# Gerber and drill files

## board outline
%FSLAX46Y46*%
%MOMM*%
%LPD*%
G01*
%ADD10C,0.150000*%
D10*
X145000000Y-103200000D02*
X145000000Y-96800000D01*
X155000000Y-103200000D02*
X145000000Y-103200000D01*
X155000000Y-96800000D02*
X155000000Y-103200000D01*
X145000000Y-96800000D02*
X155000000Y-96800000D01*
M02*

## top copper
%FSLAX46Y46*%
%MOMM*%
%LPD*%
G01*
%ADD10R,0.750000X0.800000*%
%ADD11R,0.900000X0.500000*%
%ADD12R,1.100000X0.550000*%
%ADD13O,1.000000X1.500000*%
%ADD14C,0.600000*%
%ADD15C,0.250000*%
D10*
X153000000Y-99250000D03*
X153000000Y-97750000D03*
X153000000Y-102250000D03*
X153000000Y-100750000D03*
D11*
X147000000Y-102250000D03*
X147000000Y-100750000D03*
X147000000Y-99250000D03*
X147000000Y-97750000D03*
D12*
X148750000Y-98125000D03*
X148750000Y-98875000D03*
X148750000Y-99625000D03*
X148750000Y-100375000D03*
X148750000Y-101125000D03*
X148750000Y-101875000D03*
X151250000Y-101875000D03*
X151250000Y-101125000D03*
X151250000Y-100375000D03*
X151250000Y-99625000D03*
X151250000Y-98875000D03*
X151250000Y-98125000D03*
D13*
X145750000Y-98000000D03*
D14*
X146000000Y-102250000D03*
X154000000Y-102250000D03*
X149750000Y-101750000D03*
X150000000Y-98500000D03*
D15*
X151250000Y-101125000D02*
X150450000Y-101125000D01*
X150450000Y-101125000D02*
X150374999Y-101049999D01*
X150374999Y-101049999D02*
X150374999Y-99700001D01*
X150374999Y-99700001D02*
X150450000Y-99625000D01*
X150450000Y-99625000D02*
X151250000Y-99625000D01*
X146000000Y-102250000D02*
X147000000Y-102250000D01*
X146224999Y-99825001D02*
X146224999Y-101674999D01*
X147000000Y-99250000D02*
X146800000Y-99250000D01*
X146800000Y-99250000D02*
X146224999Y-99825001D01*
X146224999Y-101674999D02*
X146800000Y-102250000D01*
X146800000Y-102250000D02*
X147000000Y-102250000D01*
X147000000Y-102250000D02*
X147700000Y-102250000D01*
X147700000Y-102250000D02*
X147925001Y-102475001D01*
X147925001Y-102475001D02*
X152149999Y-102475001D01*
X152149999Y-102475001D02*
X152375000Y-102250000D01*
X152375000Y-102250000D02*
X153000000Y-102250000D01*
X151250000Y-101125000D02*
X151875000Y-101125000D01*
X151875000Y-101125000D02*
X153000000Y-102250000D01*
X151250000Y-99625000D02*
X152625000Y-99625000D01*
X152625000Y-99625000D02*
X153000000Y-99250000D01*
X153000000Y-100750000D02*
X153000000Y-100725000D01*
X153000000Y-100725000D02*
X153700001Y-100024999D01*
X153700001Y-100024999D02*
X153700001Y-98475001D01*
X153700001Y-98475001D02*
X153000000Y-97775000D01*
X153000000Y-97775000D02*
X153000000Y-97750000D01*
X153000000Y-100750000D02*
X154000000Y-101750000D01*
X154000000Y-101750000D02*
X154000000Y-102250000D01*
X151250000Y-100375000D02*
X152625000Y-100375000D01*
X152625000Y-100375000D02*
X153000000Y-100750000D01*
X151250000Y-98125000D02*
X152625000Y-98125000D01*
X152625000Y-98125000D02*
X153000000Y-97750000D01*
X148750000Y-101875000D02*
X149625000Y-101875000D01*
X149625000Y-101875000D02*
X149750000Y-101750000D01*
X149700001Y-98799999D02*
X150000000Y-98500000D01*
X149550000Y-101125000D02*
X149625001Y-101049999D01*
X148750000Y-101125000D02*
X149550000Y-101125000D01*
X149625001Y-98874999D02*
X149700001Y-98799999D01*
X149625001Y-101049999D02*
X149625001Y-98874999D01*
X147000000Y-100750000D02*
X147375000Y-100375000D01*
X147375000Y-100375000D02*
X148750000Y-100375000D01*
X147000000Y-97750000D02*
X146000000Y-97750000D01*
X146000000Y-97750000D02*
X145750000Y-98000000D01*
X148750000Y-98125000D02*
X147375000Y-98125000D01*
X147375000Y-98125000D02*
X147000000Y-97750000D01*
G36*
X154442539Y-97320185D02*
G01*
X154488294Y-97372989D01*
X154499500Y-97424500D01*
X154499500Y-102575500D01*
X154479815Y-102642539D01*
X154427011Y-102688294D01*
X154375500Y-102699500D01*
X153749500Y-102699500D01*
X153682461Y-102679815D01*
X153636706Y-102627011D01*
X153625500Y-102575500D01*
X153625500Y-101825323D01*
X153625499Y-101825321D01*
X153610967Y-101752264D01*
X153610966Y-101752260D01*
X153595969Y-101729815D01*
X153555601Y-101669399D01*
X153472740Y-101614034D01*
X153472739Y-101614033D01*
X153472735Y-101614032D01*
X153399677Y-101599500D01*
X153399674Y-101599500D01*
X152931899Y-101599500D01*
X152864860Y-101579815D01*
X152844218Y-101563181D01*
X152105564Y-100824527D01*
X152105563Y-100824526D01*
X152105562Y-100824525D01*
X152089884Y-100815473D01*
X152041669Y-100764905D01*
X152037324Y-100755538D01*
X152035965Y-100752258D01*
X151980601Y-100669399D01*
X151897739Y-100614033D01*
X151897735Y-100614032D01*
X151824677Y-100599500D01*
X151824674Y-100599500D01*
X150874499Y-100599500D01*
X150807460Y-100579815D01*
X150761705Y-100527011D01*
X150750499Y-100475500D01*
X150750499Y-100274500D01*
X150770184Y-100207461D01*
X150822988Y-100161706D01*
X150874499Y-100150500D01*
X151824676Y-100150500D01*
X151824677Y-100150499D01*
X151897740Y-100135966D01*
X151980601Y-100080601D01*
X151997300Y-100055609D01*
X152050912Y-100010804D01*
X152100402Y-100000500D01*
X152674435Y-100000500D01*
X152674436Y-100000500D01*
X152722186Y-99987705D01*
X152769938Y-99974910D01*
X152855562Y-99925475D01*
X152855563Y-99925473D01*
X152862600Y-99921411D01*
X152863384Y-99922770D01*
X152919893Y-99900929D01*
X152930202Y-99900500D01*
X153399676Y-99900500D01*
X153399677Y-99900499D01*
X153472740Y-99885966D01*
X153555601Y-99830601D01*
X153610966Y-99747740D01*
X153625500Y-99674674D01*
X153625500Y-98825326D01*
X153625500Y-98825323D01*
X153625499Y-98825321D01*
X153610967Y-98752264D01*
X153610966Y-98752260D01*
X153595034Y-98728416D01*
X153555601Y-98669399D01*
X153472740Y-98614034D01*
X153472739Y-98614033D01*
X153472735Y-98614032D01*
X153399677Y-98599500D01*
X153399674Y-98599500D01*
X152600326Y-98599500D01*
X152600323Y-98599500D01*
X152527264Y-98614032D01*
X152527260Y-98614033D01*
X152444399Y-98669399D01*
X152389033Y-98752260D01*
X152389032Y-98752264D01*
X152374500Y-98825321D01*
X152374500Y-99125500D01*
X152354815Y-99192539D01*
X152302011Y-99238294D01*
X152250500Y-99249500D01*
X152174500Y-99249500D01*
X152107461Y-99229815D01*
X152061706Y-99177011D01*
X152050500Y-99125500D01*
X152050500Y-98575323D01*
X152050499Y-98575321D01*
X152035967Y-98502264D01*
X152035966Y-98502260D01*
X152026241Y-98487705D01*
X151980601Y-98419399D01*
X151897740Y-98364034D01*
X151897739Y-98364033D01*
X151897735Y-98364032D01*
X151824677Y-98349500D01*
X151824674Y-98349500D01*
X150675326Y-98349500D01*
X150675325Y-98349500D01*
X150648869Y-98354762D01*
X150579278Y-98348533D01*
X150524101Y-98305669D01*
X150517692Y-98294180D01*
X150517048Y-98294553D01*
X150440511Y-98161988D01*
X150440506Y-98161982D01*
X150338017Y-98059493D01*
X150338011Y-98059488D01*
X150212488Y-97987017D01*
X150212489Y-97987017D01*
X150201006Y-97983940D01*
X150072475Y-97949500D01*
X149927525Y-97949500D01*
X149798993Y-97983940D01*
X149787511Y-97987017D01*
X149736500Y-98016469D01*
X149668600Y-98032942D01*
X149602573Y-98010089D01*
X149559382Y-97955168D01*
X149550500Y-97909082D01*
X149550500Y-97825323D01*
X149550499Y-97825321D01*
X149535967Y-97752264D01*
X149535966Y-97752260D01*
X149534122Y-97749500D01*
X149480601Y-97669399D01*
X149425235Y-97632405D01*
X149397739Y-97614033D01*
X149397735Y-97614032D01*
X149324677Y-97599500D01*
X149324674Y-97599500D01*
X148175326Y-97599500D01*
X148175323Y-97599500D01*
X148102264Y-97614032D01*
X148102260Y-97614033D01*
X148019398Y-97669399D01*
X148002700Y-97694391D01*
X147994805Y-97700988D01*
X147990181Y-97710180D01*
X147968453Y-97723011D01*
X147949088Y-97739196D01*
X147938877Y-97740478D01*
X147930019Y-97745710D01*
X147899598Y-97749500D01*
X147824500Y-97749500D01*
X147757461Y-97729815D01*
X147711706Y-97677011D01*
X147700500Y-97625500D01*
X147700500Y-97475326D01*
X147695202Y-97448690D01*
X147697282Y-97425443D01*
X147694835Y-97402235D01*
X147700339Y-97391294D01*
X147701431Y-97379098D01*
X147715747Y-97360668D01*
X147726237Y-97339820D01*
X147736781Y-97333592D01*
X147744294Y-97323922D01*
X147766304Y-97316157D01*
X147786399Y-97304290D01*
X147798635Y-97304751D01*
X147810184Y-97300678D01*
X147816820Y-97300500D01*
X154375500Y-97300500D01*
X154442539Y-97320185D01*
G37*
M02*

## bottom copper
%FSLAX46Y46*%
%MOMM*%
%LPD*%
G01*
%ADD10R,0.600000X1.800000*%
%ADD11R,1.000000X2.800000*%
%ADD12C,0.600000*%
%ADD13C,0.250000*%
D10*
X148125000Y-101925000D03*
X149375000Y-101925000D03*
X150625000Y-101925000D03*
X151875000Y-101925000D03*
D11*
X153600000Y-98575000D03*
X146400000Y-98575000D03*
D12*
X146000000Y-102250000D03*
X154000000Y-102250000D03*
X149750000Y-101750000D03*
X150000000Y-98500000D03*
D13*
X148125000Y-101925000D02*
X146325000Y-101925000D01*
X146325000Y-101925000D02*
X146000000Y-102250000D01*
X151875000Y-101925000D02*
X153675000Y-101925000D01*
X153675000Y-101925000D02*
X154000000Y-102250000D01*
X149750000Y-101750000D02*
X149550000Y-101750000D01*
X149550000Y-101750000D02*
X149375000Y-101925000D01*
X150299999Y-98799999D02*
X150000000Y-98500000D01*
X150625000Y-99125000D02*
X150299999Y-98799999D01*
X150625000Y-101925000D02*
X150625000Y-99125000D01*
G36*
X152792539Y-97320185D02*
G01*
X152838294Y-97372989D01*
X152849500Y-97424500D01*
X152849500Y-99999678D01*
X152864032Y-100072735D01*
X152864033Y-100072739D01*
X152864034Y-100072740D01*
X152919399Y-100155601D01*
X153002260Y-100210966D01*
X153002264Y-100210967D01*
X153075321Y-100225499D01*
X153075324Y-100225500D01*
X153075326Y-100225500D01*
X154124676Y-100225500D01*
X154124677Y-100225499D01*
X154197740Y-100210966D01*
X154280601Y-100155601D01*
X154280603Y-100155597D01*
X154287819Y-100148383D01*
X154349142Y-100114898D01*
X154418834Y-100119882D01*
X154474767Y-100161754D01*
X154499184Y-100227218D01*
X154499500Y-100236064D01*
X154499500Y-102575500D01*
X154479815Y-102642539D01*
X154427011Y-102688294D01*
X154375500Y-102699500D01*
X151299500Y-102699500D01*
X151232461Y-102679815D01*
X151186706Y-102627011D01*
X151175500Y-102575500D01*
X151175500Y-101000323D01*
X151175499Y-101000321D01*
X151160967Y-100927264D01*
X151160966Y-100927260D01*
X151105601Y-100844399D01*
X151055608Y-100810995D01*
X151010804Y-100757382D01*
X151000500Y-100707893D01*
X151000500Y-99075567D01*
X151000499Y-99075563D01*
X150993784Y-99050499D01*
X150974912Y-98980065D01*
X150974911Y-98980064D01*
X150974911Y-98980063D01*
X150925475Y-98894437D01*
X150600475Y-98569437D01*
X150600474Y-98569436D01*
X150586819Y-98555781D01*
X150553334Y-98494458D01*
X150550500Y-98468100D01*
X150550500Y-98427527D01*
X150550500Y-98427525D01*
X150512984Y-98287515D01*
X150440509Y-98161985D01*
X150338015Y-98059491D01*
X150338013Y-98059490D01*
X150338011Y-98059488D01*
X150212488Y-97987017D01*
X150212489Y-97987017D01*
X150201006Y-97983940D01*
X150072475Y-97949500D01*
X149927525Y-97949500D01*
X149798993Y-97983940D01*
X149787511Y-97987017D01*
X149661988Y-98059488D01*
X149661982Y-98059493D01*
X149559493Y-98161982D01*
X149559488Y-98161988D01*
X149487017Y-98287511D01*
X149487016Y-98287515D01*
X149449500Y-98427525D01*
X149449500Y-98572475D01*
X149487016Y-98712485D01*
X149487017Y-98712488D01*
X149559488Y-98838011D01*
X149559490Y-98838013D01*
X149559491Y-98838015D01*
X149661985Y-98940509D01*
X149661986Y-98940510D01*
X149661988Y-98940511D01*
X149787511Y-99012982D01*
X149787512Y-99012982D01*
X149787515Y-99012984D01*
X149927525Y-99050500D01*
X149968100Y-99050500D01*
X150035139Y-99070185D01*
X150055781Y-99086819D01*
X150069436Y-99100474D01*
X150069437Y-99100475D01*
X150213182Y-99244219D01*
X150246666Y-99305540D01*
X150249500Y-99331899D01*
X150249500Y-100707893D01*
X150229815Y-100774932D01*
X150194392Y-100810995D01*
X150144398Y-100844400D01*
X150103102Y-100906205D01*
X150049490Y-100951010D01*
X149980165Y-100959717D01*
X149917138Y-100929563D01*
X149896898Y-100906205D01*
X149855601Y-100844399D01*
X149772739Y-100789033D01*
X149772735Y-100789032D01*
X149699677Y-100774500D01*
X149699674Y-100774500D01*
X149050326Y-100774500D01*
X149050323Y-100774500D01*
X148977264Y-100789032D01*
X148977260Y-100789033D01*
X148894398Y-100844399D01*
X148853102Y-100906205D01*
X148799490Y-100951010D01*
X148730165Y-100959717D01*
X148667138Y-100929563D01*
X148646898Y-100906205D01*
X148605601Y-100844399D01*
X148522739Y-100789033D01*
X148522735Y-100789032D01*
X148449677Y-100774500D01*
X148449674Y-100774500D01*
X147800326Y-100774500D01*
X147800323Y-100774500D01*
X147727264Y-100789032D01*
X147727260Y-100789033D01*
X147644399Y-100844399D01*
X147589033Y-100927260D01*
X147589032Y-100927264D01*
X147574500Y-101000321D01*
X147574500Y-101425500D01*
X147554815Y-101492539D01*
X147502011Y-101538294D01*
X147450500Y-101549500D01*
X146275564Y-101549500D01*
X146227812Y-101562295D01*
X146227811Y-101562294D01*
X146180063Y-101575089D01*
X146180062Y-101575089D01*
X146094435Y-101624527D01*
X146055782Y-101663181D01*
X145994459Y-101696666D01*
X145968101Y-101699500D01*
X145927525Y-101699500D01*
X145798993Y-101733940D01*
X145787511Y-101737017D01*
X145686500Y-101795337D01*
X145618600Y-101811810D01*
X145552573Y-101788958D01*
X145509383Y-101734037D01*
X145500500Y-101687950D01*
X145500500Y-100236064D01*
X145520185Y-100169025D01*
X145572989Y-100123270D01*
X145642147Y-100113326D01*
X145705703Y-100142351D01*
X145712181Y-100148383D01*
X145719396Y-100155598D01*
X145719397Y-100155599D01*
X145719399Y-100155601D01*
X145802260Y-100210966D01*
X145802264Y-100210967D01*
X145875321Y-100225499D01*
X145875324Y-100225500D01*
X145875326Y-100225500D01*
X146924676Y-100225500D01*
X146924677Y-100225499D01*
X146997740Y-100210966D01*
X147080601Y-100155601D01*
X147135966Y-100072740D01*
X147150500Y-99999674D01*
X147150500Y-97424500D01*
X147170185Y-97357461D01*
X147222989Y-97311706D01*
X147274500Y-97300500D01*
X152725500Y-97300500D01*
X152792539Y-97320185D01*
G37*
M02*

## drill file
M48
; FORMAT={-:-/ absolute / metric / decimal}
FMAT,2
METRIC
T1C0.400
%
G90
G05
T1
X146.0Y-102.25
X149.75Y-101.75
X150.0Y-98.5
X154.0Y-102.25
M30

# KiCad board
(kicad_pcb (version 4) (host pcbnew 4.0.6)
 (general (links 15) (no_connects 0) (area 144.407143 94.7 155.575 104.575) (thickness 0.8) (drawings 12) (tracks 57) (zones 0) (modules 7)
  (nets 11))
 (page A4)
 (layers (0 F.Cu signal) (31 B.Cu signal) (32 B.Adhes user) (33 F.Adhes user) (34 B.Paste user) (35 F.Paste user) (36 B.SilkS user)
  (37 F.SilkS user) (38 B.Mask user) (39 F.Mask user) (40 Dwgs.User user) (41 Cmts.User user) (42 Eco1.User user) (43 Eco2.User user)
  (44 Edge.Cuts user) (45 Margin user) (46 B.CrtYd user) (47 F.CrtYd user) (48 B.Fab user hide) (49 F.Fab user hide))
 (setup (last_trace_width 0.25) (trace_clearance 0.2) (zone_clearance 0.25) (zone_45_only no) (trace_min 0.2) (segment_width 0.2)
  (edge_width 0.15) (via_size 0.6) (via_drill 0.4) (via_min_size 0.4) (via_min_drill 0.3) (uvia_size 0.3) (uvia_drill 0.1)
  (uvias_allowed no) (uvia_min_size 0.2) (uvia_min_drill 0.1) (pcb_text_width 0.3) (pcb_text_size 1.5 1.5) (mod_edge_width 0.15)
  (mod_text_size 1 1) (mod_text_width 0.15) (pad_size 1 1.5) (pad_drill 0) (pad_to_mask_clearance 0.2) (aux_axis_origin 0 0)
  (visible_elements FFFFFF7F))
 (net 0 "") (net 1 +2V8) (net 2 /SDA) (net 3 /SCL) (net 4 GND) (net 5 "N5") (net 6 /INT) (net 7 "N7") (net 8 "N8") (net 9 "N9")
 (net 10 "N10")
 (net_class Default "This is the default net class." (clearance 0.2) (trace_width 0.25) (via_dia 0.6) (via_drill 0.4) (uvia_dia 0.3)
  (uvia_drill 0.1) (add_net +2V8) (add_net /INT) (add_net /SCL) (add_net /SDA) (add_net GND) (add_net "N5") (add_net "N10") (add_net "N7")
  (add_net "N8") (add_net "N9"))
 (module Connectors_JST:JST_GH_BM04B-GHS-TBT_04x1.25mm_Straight (layer B.Cu) (at 150 100.25)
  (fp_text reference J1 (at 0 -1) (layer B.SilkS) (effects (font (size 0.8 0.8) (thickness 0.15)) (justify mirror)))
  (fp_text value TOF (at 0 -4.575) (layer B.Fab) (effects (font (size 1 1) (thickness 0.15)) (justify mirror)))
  (pad 1 smd rect (at -1.875 1.675) (size 0.6 1.8) (layers B.Cu B.Paste B.Mask) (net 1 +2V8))
  (pad 2 smd rect (at -0.625 1.675) (size 0.6 1.8) (layers B.Cu B.Paste B.Mask) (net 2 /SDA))
  (pad 3 smd rect (at 0.625 1.675) (size 0.6 1.8) (layers B.Cu B.Paste B.Mask) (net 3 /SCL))
  (pad 4 smd rect (at 1.875 1.675) (size 0.6 1.8) (layers B.Cu B.Paste B.Mask) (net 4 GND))
  (pad "" smd rect (at 3.6 -1.675) (size 1 2.8) (layers B.Cu B.Paste B.Mask))
  (pad "" smd rect (at -3.6 -1.675) (size 1 2.8) (layers B.Cu B.Paste B.Mask)))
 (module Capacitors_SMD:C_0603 (layer F.Cu) (at 153 98.5 90)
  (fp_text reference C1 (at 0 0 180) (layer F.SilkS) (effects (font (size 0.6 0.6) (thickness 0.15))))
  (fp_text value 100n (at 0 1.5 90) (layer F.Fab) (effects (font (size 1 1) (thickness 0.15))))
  (pad 1 smd rect (at -0.75 0 90) (size 0.8 0.75) (layers F.Cu F.Paste F.Mask) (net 1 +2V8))
  (pad 2 smd rect (at 0.75 0 90) (size 0.8 0.75) (layers F.Cu F.Paste F.Mask) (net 4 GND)))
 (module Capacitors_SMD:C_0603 (layer F.Cu) (at 153 101.5 90)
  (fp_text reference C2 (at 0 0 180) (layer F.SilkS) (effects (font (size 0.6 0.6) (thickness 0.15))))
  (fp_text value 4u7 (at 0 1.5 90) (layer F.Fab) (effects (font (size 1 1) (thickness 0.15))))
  (pad 1 smd rect (at -0.75 0 90) (size 0.8 0.75) (layers F.Cu F.Paste F.Mask) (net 1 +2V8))
  (pad 2 smd rect (at 0.75 0 90) (size 0.8 0.75) (layers F.Cu F.Paste F.Mask) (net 4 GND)))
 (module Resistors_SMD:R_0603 (layer F.Cu) (at 147 101.5 90)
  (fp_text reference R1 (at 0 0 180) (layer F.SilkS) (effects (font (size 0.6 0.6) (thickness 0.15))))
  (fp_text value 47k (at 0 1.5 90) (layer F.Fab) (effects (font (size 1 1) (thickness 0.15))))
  (pad 1 smd rect (at -0.75 0 90) (size 0.5 0.9) (layers F.Cu F.Paste F.Mask) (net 1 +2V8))
  (pad 2 smd rect (at 0.75 0 90) (size 0.5 0.9) (layers F.Cu F.Paste F.Mask) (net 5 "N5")))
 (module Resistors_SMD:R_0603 (layer F.Cu) (at 147 98.5 90)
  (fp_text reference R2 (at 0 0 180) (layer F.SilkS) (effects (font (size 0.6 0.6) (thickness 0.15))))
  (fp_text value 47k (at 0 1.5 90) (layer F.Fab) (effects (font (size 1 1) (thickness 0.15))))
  (pad 1 smd rect (at -0.75 0 90) (size 0.5 0.9) (layers F.Cu F.Paste F.Mask) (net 1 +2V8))
  (pad 2 smd rect (at 0.75 0 90) (size 0.5 0.9) (layers F.Cu F.Paste F.Mask) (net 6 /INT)))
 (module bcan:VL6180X (layer F.Cu) (at 150 100)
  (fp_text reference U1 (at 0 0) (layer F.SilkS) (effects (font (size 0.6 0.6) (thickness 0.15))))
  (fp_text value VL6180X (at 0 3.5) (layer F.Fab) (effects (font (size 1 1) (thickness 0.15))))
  (pad 1 smd rect (at -1.25 -1.875) (size 1.1 0.55) (layers F.Cu F.Paste F.Mask) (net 6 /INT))
  (pad 2 smd rect (at -1.25 -1.125) (size 1.1 0.55) (layers F.Cu F.Paste F.Mask) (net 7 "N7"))
  (pad 3 smd rect (at -1.25 -0.375) (size 1.1 0.55) (layers F.Cu F.Paste F.Mask) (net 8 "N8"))
  (pad 4 smd rect (at -1.25 0.375) (size 1.1 0.55) (layers F.Cu F.Paste F.Mask) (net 5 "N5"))
  (pad 5 smd rect (at -1.25 1.125) (size 1.1 0.55) (layers F.Cu F.Paste F.Mask) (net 3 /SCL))
  (pad 6 smd rect (at -1.25 1.875) (size 1.1 0.55) (layers F.Cu F.Paste F.Mask) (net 2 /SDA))
  (pad 7 smd rect (at 1.25 1.875) (size 1.1 0.55) (layers F.Cu F.Paste F.Mask) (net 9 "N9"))
  (pad 8 smd rect (at 1.25 1.125) (size 1.1 0.55) (layers F.Cu F.Paste F.Mask) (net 1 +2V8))
  (pad 9 smd rect (at 1.25 0.375) (size 1.1 0.55) (layers F.Cu F.Paste F.Mask) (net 4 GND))
  (pad 10 smd rect (at 1.25 -0.375) (size 1.1 0.55) (layers F.Cu F.Paste F.Mask) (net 1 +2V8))
  (pad 11 smd rect (at 1.25 -1.125) (size 1.1 0.55) (layers F.Cu F.Paste F.Mask) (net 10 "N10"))
  (pad 12 smd rect (at 1.25 -1.875) (size 1.1 0.55) (layers F.Cu F.Paste F.Mask) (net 4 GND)))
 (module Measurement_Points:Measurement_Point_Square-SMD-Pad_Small (layer F.Cu) (at 145.75 98)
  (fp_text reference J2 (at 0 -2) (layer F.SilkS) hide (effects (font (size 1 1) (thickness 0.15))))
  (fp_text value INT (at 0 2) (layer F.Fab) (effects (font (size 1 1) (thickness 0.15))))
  (pad 1 smd oval (at 0 0) (size 1 1.5) (layers F.Cu F.Mask) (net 6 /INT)))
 (gr_line (start 145 103.2) (end 145 96.8) (layer Edge.Cuts) (width 0.15))
 (gr_line (start 155 103.2) (end 145 103.2) (layer Edge.Cuts) (width 0.15))
 (gr_line (start 155 96.8) (end 155 103.2) (layer Edge.Cuts) (width 0.15))
 (gr_line (start 145 96.8) (end 155 96.8) (layer Edge.Cuts) (width 0.15))
 (segment (start 151.25 101.125) (end 150.45 101.125) (width 0.25) (layer F.Cu) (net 1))
 (segment (start 150.45 101.125) (end 150.374999 101.049999) (width 0.25) (layer F.Cu) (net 1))
 (segment (start 150.374999 101.049999) (end 150.374999 99.700001) (width 0.25) (layer F.Cu) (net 1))
 (segment (start 150.374999 99.700001) (end 150.45 99.625) (width 0.25) (layer F.Cu) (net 1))
 (segment (start 150.45 99.625) (end 151.25 99.625) (width 0.25) (layer F.Cu) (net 1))
 (segment (start 146 102.25) (end 147 102.25) (width 0.25) (layer F.Cu) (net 1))
 (segment (start 148.125 101.925) (end 146.325 101.925) (width 0.25) (layer B.Cu) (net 1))
 (segment (start 146.325 101.925) (end 146 102.25) (width 0.25) (layer B.Cu) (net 1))
 (via (at 146 102.25) (size 0.6) (drill 0.4) (layers F.Cu B.Cu) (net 1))
 (segment (start 146.224999 99.825001) (end 146.224999 101.674999) (width 0.25) (layer F.Cu) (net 1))
 (segment (start 147 99.25) (end 146.8 99.25) (width 0.25) (layer F.Cu) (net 1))
 (segment (start 146.8 99.25) (end 146.224999 99.825001) (width 0.25) (layer F.Cu) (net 1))
 (segment (start 146.224999 101.674999) (end 146.8 102.25) (width 0.25) (layer F.Cu) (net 1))
 (segment (start 146.8 102.25) (end 147 102.25) (width 0.25) (layer F.Cu) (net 1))
 (segment (start 147 102.25) (end 147.7 102.25) (width 0.25) (layer F.Cu) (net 1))
 (segment (start 147.7 102.25) (end 147.925001 102.475001) (width 0.25) (layer F.Cu) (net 1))
 (segment (start 147.925001 102.475001) (end 152.149999 102.475001) (width 0.25) (layer F.Cu) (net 1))
 (segment (start 152.149999 102.475001) (end 152.375 102.25) (width 0.25) (layer F.Cu) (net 1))
 (segment (start 152.375 102.25) (end 153 102.25) (width 0.25) (layer F.Cu) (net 1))
 (segment (start 151.25 101.125) (end 151.875 101.125) (width 0.25) (layer F.Cu) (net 1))
 (segment (start 151.875 101.125) (end 153 102.25) (width 0.25) (layer F.Cu) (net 1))
 (segment (start 151.25 99.625) (end 152.625 99.625) (width 0.25) (layer F.Cu) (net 1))
 (segment (start 152.625 99.625) (end 153 99.25) (width 0.25) (layer F.Cu) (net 1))
 (segment (start 153 100.75) (end 153 100.725) (width 0.25) (layer F.Cu) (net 4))
 (segment (start 153 100.725) (end 153.700001 100.024999) (width 0.25) (layer F.Cu) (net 4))
 (segment (start 153.700001 100.024999) (end 153.700001 98.475001) (width 0.25) (layer F.Cu) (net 4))
 (segment (start 153.700001 98.475001) (end 153 97.775) (width 0.25) (layer F.Cu) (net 4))
 (segment (start 153 97.775) (end 153 97.75) (width 0.25) (layer F.Cu) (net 4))
 (segment (start 151.875 101.925) (end 153.675 101.925) (width 0.25) (layer B.Cu) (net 4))
 (segment (start 153.675 101.925) (end 154 102.25) (width 0.25) (layer B.Cu) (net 4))
 (segment (start 153 100.75) (end 154 101.75) (width 0.25) (layer F.Cu) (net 4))
 (via (at 154 102.25) (size 0.6) (drill 0.4) (layers F.Cu B.Cu) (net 4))
 (segment (start 154 101.75) (end 154 102.25) (width 0.25) (layer F.Cu) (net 4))
 (segment (start 151.25 100.375) (end 152.625 100.375) (width 0.25) (layer F.Cu) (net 4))
 (segment (start 152.625 100.375) (end 153 100.75) (width 0.25) (layer F.Cu) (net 4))
 (segment (start 151.25 98.125) (end 152.625 98.125) (width 0.25) (layer F.Cu) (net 4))
 (segment (start 152.625 98.125) (end 153 97.75) (width 0.25) (layer F.Cu) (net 4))
 (segment (start 149.75 101.75) (end 149.55 101.75) (width 0.25) (layer B.Cu) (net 2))
 (segment (start 149.55 101.75) (end 149.375 101.925) (width 0.25) (layer B.Cu) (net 2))
 (segment (start 148.75 101.875) (end 149.625 101.875) (width 0.25) (layer F.Cu) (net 2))
 (segment (start 149.625 101.875) (end 149.75 101.75) (width 0.25) (layer F.Cu) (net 2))
 (via (at 149.75 101.75) (size 0.6) (drill 0.4) (layers F.Cu B.Cu) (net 2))
 (segment (start 149.700001 98.799999) (end 150 98.5) (width 0.25) (layer F.Cu) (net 3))
 (segment (start 149.55 101.125) (end 149.625001 101.049999) (width 0.25) (layer F.Cu) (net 3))
 (segment (start 148.75 101.125) (end 149.55 101.125) (width 0.25) (layer F.Cu) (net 3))
 (segment (start 149.625001 98.874999) (end 149.700001 98.799999) (width 0.25) (layer F.Cu) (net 3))
 (segment (start 149.625001 101.049999) (end 149.625001 98.874999) (width 0.25) (layer F.Cu) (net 3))
 (segment (start 150.299999 98.799999) (end 150 98.5) (width 0.25) (layer B.Cu) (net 3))
 (segment (start 150.625 99.125) (end 150.299999 98.799999) (width 0.25) (layer B.Cu) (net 3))
 (segment (start 150.625 101.925) (end 150.625 99.125) (width 0.25) (layer B.Cu) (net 3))
 (via (at 150 98.5) (size 0.6) (drill 0.4) (layers F.Cu B.Cu) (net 3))
 (segment (start 147 100.75) (end 147.375 100.375) (width 0.25) (layer F.Cu) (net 5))
 (segment (start 147.375 100.375) (end 148.75 100.375) (width 0.25) (layer F.Cu) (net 5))
 (segment (start 147 97.75) (end 146 97.75) (width 0.25) (layer F.Cu) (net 6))
 (segment (start 146 97.75) (end 145.75 98) (width 0.25) (layer F.Cu) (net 6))
 (segment (start 148.75 98.125) (end 147.375 98.125) (width 0.25) (layer F.Cu) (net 6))
 (segment (start 147.375 98.125) (end 147 97.75) (width 0.25) (layer F.Cu) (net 6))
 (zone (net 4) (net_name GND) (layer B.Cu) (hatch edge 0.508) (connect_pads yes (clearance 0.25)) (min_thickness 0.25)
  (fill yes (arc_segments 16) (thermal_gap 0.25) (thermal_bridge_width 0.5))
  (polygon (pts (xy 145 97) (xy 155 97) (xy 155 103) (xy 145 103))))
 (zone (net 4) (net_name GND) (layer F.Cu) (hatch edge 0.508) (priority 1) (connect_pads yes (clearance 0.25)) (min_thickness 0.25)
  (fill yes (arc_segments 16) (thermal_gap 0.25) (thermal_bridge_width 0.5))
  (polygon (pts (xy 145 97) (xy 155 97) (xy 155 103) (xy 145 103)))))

